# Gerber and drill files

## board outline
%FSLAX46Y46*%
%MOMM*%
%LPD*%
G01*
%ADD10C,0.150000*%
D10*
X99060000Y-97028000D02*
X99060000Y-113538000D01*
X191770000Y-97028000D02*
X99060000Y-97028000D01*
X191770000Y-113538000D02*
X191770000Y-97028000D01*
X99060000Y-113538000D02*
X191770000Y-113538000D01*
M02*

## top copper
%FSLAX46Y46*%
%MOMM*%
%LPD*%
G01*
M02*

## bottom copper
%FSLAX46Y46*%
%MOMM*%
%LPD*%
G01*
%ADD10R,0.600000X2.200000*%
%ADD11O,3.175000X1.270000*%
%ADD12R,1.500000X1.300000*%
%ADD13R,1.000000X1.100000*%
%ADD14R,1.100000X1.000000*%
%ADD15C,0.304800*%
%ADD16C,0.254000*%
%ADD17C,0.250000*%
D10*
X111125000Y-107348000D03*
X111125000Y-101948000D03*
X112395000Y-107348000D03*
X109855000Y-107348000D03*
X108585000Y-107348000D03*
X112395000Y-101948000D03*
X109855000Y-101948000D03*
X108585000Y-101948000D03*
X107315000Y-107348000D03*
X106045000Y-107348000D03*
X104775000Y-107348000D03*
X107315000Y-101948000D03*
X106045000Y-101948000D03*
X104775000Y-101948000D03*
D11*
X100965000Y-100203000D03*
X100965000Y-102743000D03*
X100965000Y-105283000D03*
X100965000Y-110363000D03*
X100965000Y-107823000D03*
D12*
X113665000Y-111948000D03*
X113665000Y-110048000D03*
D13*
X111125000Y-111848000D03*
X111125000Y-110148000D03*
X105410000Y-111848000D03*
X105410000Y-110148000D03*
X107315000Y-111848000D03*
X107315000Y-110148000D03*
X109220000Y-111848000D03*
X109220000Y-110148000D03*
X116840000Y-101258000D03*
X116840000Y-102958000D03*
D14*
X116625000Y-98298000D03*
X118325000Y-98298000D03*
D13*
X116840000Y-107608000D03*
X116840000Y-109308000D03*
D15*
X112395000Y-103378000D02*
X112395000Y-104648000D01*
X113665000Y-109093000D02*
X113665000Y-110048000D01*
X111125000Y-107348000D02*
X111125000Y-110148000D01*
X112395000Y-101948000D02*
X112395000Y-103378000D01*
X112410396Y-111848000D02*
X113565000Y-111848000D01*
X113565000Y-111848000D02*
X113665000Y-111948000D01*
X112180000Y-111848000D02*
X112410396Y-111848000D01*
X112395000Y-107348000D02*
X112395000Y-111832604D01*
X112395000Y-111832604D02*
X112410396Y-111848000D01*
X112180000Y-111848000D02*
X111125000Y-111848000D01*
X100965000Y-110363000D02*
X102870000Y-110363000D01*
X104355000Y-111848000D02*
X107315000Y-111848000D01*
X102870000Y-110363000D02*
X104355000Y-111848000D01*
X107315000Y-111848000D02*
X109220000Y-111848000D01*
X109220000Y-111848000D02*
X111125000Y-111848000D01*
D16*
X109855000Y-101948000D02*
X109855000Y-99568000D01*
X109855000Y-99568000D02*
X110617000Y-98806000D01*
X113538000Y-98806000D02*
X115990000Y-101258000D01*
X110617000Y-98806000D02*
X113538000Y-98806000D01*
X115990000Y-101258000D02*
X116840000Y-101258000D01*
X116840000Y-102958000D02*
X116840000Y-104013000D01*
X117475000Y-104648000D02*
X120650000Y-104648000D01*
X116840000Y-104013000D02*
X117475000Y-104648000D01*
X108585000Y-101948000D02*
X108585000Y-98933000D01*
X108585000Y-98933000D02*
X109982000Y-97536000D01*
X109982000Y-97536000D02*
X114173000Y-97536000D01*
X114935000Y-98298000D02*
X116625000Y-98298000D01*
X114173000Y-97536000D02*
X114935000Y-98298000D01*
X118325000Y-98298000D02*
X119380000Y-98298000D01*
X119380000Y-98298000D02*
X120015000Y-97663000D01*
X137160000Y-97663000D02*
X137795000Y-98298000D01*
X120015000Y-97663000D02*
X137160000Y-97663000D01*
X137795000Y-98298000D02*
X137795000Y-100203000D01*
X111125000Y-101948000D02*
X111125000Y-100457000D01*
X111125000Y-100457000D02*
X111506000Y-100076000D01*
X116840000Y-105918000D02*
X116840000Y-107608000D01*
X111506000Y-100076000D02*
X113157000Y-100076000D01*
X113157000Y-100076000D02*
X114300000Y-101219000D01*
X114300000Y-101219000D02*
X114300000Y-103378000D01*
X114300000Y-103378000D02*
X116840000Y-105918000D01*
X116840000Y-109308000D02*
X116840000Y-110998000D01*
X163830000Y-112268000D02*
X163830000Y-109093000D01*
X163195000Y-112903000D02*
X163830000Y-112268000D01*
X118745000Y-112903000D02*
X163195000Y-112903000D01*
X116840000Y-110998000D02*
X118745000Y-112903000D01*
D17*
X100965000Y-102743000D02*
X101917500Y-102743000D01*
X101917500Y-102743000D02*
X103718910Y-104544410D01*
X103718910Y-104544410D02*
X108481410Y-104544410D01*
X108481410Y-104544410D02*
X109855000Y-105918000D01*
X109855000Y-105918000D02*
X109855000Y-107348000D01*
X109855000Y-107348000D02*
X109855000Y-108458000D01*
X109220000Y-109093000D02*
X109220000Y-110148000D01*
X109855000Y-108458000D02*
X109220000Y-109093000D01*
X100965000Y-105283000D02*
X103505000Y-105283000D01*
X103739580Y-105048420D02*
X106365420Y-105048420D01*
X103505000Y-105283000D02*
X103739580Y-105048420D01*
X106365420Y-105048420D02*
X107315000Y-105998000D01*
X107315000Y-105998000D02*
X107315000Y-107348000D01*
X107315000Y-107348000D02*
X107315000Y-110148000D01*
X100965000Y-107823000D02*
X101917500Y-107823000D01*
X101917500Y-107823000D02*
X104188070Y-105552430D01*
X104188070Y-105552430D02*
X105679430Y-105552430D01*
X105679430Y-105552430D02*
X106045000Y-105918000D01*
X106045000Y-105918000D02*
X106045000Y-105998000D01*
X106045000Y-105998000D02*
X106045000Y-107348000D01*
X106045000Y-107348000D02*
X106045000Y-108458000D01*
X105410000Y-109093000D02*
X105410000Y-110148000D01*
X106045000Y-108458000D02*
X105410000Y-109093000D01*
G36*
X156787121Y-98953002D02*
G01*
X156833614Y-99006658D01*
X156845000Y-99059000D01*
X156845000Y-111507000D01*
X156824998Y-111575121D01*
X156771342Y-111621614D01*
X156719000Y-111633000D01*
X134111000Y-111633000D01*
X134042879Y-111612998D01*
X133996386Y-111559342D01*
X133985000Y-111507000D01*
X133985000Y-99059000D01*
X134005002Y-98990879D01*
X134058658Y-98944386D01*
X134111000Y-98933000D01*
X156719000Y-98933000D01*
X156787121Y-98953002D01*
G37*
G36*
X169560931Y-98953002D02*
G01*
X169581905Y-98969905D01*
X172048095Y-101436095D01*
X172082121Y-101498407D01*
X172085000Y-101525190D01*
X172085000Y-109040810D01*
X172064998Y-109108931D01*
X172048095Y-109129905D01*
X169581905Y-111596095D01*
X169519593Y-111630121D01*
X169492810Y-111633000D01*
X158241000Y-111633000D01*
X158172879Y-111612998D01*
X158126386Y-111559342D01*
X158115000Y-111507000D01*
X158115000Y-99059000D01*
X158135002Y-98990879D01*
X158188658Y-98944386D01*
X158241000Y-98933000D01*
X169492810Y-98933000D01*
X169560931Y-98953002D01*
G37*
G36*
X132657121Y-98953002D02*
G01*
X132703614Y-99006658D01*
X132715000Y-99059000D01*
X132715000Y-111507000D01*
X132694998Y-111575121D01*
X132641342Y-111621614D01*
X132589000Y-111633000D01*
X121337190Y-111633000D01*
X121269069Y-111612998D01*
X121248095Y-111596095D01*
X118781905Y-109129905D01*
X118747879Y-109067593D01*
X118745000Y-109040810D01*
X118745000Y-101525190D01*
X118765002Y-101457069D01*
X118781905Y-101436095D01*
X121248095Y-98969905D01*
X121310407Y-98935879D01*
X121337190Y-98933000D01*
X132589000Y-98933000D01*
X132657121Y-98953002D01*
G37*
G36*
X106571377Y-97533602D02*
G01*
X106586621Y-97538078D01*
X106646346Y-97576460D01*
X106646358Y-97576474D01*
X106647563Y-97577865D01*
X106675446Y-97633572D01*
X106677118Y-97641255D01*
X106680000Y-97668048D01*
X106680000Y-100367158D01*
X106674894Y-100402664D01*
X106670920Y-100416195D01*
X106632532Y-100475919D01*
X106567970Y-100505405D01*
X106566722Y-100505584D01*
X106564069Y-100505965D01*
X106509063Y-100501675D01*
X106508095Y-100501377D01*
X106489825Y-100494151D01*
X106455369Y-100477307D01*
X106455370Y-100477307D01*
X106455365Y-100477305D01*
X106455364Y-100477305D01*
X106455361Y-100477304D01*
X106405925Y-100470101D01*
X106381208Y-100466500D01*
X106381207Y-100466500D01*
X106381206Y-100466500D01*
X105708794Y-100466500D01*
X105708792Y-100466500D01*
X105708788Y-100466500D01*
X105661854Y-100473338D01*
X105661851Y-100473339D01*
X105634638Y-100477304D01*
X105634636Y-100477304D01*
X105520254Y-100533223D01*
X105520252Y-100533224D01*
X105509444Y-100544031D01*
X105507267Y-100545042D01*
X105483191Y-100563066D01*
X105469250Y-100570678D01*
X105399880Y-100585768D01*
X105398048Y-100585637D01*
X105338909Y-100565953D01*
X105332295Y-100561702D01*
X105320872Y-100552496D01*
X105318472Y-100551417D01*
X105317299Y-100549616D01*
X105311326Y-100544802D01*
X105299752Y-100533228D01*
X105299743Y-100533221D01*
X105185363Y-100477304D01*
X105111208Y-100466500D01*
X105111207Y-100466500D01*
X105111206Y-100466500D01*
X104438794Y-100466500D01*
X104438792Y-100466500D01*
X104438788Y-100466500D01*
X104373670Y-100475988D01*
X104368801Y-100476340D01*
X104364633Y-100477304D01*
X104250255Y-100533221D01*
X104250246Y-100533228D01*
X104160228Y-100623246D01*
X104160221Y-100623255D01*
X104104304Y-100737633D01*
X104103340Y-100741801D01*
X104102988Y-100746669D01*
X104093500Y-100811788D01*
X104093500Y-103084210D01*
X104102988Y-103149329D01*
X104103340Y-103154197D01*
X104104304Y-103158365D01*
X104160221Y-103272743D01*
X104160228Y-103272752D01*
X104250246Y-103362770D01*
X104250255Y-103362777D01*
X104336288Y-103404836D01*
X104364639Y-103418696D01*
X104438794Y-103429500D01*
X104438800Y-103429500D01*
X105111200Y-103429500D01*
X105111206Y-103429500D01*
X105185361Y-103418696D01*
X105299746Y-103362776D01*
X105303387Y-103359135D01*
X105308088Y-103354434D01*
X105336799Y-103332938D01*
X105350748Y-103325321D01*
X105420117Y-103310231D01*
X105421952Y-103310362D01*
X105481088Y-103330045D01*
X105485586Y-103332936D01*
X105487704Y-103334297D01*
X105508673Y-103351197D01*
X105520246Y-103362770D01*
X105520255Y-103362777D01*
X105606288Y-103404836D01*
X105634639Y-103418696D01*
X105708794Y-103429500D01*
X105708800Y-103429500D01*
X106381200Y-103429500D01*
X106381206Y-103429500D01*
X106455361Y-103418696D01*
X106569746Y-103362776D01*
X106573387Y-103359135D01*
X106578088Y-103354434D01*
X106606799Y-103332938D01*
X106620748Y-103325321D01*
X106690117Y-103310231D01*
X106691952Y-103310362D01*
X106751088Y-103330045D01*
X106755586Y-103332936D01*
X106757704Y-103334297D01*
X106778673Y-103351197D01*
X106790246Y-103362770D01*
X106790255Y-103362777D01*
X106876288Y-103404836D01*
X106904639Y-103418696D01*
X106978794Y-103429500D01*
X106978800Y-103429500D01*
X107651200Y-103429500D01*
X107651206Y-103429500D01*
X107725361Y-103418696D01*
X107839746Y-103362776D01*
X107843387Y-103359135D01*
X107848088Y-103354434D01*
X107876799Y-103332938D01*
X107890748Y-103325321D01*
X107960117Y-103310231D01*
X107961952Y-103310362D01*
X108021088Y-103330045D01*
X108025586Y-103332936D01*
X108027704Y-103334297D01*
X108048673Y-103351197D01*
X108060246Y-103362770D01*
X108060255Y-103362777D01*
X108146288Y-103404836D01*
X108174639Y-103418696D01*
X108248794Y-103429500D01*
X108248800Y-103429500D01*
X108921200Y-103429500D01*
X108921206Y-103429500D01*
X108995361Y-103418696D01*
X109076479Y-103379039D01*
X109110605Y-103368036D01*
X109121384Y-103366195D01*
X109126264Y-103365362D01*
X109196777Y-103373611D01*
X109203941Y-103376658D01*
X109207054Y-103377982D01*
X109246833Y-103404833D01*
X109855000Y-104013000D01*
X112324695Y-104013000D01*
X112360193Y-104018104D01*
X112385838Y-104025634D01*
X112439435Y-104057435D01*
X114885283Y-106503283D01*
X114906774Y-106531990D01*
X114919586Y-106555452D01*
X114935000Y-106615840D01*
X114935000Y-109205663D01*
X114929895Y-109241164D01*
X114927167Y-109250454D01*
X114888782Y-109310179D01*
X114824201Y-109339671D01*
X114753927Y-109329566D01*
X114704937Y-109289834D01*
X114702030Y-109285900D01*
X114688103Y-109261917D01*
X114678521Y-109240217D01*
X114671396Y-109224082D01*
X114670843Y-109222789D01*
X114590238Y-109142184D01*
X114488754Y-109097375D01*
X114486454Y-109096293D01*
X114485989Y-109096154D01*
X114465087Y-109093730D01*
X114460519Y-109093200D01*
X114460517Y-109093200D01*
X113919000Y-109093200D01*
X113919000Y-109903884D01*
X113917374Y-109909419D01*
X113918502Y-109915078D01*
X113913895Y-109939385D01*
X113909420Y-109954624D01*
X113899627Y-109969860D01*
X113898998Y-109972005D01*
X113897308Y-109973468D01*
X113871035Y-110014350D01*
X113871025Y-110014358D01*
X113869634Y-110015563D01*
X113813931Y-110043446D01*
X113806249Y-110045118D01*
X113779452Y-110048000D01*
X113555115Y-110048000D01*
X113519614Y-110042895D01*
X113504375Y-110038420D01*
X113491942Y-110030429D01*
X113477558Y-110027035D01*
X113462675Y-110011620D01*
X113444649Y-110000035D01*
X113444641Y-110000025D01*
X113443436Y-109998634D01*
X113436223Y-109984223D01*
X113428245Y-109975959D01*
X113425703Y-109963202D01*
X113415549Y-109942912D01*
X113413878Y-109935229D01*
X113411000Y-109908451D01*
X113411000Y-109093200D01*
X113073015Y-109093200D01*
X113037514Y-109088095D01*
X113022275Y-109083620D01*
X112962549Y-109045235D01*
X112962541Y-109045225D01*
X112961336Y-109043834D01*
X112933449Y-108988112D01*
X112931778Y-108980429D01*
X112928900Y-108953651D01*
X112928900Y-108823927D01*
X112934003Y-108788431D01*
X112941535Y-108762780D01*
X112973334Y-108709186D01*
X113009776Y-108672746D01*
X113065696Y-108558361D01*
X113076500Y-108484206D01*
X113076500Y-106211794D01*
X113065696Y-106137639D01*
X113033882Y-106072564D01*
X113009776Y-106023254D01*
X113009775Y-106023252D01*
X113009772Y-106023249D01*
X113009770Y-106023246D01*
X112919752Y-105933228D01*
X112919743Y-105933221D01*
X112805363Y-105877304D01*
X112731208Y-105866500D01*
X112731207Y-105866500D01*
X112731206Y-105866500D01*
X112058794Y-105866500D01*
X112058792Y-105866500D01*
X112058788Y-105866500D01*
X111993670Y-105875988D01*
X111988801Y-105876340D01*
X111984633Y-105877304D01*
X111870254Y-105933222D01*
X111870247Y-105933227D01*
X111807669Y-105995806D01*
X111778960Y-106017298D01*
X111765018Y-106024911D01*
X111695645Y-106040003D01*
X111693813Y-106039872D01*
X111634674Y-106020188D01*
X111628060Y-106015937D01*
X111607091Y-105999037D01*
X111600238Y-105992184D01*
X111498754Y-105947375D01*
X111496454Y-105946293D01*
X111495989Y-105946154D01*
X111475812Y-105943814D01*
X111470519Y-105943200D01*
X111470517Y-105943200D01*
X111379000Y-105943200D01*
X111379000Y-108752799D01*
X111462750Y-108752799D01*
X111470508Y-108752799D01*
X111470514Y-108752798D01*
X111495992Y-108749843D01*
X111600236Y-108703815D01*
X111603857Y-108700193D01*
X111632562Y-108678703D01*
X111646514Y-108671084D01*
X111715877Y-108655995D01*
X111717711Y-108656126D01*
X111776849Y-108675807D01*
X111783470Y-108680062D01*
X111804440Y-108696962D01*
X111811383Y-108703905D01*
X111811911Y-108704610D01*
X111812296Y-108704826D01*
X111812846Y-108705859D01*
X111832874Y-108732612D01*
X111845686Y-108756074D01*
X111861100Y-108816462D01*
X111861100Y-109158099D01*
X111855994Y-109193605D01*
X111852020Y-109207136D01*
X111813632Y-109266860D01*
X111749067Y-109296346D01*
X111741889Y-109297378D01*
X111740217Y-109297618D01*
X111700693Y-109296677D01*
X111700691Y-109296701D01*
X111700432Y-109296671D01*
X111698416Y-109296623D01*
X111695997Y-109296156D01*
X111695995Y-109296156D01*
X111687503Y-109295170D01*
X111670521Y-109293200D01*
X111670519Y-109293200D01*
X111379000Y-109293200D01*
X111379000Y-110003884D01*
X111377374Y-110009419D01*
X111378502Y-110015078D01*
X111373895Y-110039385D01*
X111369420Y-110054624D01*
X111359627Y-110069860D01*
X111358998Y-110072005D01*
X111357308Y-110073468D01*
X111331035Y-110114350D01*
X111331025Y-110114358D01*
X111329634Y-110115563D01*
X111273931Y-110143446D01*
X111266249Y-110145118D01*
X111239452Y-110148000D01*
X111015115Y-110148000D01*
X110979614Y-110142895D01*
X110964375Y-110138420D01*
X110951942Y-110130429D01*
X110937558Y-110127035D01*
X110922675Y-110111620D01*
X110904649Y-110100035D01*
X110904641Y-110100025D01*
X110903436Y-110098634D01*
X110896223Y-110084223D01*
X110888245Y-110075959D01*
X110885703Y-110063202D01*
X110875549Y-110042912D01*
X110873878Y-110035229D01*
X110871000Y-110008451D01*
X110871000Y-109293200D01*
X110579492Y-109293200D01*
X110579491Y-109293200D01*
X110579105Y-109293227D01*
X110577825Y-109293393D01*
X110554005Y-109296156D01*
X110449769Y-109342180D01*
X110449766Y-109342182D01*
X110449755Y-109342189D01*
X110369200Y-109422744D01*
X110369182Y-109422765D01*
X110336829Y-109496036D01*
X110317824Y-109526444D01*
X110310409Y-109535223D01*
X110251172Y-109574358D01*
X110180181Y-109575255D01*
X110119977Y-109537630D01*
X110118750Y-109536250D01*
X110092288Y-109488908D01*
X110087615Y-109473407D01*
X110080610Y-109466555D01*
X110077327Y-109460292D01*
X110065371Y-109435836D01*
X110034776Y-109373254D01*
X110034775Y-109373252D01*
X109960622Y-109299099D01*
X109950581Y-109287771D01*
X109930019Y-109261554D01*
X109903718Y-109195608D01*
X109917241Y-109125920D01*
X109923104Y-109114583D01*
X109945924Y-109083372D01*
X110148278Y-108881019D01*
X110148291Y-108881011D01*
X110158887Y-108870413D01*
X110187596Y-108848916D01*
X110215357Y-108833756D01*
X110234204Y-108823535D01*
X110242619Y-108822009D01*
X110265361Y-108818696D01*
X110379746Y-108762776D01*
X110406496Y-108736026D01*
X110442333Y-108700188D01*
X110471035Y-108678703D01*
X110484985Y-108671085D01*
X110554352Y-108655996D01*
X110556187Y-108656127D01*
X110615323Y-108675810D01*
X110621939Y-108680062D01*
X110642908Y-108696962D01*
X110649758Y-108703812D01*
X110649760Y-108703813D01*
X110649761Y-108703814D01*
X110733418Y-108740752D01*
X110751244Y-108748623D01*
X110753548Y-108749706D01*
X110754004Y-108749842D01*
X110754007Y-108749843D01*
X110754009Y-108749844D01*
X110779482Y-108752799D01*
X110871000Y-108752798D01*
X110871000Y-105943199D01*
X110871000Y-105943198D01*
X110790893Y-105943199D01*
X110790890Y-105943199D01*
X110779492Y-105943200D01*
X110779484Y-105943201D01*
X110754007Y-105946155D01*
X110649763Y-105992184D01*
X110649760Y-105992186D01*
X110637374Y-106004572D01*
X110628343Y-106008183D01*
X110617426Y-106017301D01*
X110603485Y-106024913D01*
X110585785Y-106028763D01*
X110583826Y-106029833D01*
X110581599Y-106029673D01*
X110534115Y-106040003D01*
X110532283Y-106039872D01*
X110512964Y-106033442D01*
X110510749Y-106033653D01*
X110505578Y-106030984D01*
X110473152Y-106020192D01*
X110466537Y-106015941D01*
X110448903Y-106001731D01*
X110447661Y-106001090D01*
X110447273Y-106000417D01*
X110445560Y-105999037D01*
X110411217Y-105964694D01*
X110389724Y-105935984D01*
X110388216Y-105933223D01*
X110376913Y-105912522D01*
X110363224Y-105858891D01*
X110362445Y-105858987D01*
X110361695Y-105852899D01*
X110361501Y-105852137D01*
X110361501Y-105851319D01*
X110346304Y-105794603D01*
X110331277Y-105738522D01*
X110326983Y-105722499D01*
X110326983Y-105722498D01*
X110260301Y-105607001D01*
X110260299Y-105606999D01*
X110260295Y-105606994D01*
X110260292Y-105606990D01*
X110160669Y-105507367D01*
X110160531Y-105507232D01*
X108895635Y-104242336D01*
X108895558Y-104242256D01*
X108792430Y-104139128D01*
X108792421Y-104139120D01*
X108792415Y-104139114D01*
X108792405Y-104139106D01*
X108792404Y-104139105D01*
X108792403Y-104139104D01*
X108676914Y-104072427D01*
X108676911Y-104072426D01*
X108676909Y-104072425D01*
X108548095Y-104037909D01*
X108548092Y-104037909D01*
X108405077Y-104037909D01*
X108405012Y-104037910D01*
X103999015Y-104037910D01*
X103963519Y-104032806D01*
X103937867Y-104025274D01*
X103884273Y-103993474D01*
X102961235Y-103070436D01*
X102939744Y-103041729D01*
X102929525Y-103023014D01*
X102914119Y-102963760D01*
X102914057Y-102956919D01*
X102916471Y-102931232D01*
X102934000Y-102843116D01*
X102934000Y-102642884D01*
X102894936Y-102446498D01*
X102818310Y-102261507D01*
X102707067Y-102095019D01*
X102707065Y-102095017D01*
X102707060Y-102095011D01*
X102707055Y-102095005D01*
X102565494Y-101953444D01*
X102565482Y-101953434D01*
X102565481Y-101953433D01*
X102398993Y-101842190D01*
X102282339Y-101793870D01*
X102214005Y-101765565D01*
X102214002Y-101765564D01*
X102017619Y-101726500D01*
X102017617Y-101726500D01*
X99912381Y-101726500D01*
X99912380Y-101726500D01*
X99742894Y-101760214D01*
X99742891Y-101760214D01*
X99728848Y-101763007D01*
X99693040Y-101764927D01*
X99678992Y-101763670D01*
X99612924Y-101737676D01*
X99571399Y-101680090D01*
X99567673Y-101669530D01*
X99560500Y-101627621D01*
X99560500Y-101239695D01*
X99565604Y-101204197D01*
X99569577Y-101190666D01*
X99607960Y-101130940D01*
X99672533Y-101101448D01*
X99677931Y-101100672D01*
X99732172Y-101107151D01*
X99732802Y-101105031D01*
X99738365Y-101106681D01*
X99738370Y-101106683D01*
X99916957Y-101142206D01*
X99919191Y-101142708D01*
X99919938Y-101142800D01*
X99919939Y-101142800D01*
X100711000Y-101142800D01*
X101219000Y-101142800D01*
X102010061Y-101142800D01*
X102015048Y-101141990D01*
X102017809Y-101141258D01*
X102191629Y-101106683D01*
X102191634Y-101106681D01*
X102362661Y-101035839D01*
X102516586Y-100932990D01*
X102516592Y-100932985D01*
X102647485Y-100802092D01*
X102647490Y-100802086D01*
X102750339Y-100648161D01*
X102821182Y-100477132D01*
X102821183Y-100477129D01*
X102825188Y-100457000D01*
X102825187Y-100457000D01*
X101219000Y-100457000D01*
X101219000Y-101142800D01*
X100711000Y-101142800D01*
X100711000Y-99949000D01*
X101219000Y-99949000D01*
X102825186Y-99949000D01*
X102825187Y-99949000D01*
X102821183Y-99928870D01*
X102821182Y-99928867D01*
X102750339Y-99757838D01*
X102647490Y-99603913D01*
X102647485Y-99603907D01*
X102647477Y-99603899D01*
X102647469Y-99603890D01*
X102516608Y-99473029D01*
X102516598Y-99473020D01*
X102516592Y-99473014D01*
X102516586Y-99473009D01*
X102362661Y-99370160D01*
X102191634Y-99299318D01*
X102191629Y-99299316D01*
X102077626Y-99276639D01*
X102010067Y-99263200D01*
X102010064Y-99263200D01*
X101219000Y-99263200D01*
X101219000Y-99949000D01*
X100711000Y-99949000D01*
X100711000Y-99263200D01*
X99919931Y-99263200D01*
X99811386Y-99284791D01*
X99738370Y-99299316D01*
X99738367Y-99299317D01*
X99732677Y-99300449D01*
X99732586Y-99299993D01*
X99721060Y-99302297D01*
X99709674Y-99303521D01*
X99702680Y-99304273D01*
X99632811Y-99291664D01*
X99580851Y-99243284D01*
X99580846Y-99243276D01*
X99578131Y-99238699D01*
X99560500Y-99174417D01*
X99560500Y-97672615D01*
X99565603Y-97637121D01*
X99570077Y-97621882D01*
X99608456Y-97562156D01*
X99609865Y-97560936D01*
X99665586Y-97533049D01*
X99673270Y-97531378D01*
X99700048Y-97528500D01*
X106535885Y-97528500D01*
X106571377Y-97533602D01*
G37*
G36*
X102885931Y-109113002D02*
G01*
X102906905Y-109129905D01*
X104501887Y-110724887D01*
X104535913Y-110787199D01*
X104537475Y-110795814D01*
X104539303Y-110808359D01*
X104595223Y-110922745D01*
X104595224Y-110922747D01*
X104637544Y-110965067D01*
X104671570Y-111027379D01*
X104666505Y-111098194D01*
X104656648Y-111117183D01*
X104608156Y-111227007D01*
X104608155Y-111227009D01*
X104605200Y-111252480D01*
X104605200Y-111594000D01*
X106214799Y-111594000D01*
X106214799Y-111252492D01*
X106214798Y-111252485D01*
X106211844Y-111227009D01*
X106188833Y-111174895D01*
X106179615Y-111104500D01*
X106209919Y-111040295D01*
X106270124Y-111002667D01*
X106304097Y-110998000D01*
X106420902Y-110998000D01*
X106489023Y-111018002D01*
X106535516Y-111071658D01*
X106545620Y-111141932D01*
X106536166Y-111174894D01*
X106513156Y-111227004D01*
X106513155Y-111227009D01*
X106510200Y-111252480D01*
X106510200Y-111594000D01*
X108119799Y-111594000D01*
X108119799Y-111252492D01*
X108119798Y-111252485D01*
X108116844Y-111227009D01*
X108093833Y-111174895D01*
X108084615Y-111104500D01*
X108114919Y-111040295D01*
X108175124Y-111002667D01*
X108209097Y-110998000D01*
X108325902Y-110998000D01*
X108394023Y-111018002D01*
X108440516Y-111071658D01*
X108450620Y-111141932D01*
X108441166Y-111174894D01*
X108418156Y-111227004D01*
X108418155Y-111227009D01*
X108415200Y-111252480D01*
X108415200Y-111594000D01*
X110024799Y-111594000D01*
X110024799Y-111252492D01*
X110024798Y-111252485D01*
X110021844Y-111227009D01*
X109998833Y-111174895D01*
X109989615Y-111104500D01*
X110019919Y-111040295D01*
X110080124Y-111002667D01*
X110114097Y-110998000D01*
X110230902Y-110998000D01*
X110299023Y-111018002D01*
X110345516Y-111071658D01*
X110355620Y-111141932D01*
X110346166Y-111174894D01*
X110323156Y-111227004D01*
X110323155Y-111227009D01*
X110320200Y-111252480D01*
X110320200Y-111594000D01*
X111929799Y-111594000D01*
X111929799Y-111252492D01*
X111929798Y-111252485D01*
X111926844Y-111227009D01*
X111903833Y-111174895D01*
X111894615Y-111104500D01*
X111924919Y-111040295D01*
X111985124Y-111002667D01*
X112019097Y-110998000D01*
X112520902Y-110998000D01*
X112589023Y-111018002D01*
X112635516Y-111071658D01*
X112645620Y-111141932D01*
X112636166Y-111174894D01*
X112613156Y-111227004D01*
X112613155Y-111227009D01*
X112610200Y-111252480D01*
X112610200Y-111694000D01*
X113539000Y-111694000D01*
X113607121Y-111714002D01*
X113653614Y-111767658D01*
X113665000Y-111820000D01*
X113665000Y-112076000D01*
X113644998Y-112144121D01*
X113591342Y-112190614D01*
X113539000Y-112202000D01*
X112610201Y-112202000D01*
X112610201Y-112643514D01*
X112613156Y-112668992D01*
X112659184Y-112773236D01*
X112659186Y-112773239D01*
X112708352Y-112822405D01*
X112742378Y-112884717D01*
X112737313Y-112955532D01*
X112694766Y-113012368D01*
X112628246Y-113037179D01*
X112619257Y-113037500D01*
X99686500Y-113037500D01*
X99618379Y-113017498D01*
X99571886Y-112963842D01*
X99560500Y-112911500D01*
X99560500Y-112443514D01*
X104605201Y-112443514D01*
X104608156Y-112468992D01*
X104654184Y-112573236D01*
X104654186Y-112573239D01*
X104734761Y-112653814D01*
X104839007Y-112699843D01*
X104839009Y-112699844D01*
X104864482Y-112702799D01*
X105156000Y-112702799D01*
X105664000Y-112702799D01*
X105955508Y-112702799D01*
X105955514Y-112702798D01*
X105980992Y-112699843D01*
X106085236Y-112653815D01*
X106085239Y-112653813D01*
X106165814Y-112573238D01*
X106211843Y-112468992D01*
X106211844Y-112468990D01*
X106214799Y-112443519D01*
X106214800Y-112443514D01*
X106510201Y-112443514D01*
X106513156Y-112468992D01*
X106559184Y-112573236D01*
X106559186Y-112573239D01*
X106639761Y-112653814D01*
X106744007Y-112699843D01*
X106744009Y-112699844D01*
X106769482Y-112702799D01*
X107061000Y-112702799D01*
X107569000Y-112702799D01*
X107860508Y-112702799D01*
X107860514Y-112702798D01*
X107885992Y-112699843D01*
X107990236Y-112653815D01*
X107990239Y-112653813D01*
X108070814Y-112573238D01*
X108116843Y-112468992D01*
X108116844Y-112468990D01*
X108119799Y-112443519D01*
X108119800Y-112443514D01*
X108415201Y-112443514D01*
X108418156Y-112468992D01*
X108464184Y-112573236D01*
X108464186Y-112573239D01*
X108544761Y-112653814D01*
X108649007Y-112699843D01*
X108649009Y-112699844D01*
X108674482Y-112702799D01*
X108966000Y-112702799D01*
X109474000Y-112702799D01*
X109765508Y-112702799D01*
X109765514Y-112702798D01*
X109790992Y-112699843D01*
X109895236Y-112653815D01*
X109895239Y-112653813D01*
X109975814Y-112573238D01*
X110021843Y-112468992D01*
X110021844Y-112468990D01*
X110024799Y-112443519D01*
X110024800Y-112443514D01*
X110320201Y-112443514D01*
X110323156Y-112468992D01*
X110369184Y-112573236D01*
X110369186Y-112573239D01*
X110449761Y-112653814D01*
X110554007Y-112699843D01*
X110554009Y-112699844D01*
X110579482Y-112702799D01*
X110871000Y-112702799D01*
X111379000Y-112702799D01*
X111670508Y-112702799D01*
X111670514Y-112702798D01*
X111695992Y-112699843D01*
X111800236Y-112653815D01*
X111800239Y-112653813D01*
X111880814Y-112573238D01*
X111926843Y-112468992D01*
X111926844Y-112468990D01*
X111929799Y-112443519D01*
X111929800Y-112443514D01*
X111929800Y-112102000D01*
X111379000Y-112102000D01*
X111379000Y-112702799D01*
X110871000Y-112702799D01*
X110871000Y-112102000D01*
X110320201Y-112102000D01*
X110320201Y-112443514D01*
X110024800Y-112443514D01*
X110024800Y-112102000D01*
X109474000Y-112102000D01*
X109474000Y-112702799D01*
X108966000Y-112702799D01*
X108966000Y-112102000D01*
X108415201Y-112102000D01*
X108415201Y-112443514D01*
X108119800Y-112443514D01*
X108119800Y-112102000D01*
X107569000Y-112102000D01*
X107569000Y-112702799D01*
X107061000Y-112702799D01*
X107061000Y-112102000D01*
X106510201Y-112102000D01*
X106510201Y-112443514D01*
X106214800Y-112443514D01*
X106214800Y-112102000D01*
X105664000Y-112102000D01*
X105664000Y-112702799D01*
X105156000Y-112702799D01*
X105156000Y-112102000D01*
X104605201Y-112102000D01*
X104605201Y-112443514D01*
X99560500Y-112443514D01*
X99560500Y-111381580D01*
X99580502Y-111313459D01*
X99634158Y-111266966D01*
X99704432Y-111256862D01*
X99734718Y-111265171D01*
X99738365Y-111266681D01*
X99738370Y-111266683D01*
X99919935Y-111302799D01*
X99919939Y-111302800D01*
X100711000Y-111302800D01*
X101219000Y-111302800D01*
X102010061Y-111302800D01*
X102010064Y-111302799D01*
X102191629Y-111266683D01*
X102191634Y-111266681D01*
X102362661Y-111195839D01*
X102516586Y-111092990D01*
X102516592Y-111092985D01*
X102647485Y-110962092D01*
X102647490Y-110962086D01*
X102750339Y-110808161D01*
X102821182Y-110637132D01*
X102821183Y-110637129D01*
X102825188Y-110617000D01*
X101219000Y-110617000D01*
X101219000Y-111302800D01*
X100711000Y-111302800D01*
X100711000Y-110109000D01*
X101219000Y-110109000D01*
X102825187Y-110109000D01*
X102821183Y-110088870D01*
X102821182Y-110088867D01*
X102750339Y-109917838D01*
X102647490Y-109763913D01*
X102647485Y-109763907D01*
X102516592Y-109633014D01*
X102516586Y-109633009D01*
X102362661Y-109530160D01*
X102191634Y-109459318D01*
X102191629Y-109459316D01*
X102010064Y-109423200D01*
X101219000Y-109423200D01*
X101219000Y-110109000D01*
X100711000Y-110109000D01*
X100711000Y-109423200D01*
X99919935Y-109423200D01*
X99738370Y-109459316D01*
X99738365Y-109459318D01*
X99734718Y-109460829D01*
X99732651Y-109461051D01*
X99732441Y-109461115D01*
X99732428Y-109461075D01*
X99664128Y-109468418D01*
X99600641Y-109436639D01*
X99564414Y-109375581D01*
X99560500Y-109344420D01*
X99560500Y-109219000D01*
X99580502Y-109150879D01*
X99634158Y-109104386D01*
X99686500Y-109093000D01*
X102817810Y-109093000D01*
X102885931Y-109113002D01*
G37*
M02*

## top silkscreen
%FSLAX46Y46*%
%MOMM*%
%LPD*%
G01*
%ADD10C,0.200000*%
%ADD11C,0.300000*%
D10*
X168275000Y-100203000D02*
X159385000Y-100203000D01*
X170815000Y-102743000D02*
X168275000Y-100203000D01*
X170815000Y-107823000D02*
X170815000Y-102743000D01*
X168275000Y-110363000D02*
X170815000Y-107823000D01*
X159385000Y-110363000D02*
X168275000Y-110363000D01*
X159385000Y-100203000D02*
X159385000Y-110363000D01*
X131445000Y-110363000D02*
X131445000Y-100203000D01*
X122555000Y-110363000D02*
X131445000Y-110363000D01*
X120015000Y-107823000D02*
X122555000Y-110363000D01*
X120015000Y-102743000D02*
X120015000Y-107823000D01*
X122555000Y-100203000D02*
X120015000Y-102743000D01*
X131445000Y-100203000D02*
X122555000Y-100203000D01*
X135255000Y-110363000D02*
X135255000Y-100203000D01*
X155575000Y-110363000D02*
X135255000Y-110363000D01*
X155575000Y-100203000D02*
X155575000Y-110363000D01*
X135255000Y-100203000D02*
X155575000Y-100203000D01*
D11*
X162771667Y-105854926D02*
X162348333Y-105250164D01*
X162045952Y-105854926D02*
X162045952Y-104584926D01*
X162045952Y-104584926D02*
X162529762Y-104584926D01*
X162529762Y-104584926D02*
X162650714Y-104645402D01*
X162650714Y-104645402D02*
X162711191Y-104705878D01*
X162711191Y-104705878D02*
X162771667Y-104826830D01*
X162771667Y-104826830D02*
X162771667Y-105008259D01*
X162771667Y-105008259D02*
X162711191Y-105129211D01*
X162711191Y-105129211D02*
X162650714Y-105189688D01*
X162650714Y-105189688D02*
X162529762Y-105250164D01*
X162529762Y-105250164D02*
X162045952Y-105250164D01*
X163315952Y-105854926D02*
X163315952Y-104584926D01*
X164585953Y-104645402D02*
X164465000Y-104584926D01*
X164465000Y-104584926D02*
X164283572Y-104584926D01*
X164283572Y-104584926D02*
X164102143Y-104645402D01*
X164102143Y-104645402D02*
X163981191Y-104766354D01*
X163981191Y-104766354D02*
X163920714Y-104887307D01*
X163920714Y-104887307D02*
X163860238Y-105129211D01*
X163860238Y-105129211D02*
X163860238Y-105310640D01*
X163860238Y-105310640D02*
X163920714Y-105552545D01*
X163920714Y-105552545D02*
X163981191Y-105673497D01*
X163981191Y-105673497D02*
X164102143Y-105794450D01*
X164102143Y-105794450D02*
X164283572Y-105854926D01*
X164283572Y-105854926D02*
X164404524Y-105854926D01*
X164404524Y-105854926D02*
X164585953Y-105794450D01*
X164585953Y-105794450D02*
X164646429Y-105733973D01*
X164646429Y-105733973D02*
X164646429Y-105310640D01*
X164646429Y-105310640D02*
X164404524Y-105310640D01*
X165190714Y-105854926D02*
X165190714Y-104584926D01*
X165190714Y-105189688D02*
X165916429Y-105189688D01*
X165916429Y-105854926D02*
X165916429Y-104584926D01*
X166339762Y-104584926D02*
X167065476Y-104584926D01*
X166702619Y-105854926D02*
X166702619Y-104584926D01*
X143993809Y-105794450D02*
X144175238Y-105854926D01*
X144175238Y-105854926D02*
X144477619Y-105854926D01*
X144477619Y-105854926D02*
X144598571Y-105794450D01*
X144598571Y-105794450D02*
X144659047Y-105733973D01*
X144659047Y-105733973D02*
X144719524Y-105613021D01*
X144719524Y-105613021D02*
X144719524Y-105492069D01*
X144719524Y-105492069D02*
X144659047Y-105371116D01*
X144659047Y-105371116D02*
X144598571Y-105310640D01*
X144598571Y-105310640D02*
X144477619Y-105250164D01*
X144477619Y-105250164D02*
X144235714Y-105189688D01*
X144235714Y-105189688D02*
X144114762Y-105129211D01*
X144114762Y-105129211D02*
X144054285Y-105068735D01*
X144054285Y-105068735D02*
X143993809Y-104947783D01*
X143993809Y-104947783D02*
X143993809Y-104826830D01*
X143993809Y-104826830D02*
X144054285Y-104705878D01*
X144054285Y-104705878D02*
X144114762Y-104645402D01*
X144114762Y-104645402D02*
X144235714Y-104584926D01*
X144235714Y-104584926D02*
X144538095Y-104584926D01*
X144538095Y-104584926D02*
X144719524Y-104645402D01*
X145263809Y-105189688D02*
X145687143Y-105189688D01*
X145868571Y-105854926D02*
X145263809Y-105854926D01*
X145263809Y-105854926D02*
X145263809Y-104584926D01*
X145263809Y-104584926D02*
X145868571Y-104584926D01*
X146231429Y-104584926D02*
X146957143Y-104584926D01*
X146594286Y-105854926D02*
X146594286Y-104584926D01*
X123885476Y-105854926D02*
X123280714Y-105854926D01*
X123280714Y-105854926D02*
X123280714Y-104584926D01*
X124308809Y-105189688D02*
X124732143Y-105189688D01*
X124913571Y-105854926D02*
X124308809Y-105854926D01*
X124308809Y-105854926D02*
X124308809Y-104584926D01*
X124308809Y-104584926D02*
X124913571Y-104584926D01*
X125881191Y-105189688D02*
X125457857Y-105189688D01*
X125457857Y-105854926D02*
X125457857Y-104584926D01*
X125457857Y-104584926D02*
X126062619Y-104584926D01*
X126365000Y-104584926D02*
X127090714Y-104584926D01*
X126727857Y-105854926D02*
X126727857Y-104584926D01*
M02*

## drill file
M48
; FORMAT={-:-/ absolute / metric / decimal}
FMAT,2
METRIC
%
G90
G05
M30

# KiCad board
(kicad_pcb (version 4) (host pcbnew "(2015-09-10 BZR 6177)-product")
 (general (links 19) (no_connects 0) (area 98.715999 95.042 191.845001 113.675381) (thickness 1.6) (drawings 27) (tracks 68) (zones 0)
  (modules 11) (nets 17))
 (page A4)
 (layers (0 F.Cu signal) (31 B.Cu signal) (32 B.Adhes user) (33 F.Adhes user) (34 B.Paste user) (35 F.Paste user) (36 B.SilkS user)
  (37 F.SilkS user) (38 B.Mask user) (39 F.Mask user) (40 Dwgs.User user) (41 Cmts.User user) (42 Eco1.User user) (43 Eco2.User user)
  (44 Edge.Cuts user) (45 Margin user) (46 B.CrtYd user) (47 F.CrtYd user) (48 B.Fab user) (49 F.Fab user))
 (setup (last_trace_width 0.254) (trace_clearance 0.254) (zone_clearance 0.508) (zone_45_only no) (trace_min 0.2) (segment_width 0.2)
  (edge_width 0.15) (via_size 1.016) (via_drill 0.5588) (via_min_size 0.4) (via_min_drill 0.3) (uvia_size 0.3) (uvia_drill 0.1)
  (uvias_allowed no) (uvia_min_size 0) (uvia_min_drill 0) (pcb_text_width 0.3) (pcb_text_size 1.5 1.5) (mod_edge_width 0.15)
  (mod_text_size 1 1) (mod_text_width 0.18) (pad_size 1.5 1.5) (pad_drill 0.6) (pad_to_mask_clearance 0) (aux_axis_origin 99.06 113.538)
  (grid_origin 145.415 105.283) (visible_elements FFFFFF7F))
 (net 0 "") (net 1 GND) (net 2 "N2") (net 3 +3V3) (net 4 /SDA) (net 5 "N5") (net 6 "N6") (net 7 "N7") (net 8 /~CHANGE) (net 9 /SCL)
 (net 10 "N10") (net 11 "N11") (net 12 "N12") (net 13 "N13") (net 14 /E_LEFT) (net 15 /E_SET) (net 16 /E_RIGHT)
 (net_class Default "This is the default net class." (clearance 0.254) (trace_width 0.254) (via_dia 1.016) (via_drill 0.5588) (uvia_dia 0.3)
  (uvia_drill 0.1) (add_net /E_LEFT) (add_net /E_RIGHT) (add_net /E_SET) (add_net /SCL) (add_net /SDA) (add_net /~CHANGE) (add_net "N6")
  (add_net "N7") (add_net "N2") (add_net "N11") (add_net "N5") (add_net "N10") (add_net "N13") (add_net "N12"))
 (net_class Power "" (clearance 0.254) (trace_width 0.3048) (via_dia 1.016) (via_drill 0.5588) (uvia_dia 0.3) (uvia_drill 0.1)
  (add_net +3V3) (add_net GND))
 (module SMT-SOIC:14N (layer B.Cu) (at 108.585 104.648 180)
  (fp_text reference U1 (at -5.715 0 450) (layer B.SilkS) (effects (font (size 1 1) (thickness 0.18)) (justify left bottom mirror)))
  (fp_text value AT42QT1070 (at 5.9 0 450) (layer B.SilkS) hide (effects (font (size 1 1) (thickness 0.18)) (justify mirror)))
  (pad 2 smd rect (at -2.54 -2.7 180) (size 0.6 2.2) (layers B.Cu B.Paste B.Mask) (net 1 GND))
  (pad 13 smd rect (at -2.54 2.7 180) (size 0.6 2.2) (layers B.Cu B.Paste B.Mask) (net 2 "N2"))
  (pad 1 smd rect (at -3.81 -2.7 180) (size 0.6 2.2) (layers B.Cu B.Paste B.Mask) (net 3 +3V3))
  (pad 3 smd rect (at -1.27 -2.7 180) (size 0.6 2.2) (layers B.Cu B.Paste B.Mask) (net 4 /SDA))
  (pad 4 smd rect (at 0 -2.7 180) (size 0.6 2.2) (layers B.Cu B.Paste B.Mask) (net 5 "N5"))
  (pad 14 smd rect (at -3.81 2.7 180) (size 0.6 2.2) (layers B.Cu B.Paste B.Mask) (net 1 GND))
  (pad 12 smd rect (at -1.27 2.7 180) (size 0.6 2.2) (layers B.Cu B.Paste B.Mask) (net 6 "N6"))
  (pad 11 smd rect (at 0 2.7 180) (size 0.6 2.2) (layers B.Cu B.Paste B.Mask) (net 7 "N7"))
  (pad 5 smd rect (at 1.27 -2.7 180) (size 0.6 2.2) (layers B.Cu B.Paste B.Mask) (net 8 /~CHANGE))
  (pad 6 smd rect (at 2.54 -2.7 180) (size 0.6 2.2) (layers B.Cu B.Paste B.Mask) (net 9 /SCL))
  (pad 7 smd rect (at 3.81 -2.7 180) (size 0.6 2.2) (layers B.Cu B.Paste B.Mask) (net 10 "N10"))
  (pad 10 smd rect (at 1.27 2.7 180) (size 0.6 2.2) (layers B.Cu B.Paste B.Mask) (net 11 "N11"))
  (pad 9 smd rect (at 2.54 2.7 180) (size 0.6 2.2) (layers B.Cu B.Paste B.Mask) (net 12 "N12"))
  (pad 8 smd rect (at 3.81 2.7 180) (size 0.6 2.2) (layers B.Cu B.Paste B.Mask) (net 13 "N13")))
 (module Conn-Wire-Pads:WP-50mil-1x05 (layer B.Cu) (at 100.965 105.283 270)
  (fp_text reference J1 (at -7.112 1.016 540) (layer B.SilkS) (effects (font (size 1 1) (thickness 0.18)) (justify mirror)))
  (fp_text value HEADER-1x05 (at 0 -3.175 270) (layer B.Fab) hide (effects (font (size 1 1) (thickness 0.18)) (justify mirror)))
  (pad 1 smd oval (at -5.08 0 270) (size 1.27 3.175) (layers B.Cu B.Paste B.Mask) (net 1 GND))
  (pad 2 smd oval (at -2.54 0 270) (size 1.27 3.175) (layers B.Cu B.Paste B.Mask) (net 4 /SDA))
  (pad 3 smd oval (at 0 0 270) (size 1.27 3.175) (layers B.Cu B.Paste B.Mask) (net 8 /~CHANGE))
  (pad 5 smd oval (at 5.08 0 270) (size 1.27 3.175) (layers B.Cu B.Paste B.Mask) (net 3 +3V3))
  (pad 4 smd oval (at 2.54 0 270) (size 1.27 3.175) (layers B.Cu B.Paste B.Mask) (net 9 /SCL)))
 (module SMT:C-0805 (layer B.Cu) (at 113.665 110.998 90)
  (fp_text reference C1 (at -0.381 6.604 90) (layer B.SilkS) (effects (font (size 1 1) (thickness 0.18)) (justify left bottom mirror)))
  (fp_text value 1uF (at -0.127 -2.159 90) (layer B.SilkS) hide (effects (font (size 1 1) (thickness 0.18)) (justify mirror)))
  (pad 1 smd rect (at -0.95 0 90) (size 1.3 1.5) (layers B.Cu B.Paste B.Mask) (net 3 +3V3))
  (pad 2 smd rect (at 0.95 0 90) (size 1.3 1.5) (layers B.Cu B.Paste B.Mask) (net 1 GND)))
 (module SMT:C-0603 (layer B.Cu) (at 111.125 110.998 90)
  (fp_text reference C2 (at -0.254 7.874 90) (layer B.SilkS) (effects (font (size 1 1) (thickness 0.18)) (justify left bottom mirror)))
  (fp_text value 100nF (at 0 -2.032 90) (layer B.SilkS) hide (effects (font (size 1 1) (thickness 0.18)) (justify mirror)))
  (pad 1 smd rect (at -0.85 0 90) (size 1.1 1) (layers B.Cu B.Paste B.Mask) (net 3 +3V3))
  (pad 2 smd rect (at 0.85 0 90) (size 1.1 1) (layers B.Cu B.Paste B.Mask) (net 1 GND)))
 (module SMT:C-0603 (layer B.Cu) (at 105.41 110.998 90)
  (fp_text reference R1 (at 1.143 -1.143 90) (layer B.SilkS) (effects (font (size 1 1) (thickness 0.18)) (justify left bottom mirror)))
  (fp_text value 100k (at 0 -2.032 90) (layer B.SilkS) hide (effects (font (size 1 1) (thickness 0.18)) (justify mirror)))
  (pad 1 smd rect (at -0.85 0 90) (size 1.1 1) (layers B.Cu B.Paste B.Mask) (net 3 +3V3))
  (pad 2 smd rect (at 0.85 0 90) (size 1.1 1) (layers B.Cu B.Paste B.Mask) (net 9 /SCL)))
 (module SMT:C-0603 (layer B.Cu) (at 107.315 110.998 90)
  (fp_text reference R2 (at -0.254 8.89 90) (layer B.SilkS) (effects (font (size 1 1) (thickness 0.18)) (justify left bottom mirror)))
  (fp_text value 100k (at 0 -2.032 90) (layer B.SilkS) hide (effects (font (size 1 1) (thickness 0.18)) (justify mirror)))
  (pad 1 smd rect (at -0.85 0 90) (size 1.1 1) (layers B.Cu B.Paste B.Mask) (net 3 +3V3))
  (pad 2 smd rect (at 0.85 0 90) (size 1.1 1) (layers B.Cu B.Paste B.Mask) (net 8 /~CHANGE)))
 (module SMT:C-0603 (layer B.Cu) (at 109.22 110.998 90)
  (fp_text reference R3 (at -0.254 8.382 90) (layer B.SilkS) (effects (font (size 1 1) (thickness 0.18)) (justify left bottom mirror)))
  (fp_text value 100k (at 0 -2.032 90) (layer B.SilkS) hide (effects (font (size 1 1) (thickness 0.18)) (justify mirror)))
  (pad 1 smd rect (at -0.85 0 90) (size 1.1 1) (layers B.Cu B.Paste B.Mask) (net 3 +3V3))
  (pad 2 smd rect (at 0.85 0 90) (size 1.1 1) (layers B.Cu B.Paste B.Mask) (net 4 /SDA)))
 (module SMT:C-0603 (layer B.Cu) (at 116.84 102.108 270)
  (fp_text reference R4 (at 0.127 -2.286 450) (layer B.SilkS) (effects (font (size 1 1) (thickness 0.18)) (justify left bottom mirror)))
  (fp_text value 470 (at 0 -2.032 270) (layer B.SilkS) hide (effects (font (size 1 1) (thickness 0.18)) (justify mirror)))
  (pad 1 smd rect (at -0.85 0 270) (size 1.1 1) (layers B.Cu B.Paste B.Mask) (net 6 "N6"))
  (pad 2 smd rect (at 0.85 0 270) (size 1.1 1) (layers B.Cu B.Paste B.Mask) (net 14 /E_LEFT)))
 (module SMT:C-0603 (layer B.Cu) (at 117.475 98.298)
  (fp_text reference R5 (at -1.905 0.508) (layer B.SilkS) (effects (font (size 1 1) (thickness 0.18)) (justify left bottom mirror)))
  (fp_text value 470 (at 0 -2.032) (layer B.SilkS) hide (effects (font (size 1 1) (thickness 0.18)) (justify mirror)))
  (pad 1 smd rect (at -0.85 0) (size 1.1 1) (layers B.Cu B.Paste B.Mask) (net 7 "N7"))
  (pad 2 smd rect (at 0.85 0) (size 1.1 1) (layers B.Cu B.Paste B.Mask) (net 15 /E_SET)))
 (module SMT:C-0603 (layer B.Cu) (at 116.84 108.458 270)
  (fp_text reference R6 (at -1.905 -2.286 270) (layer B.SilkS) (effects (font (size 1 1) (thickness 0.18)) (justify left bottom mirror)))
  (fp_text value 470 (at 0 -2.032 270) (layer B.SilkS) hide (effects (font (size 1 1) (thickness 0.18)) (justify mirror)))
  (pad 1 smd rect (at -0.85 0 270) (size 1.1 1) (layers B.Cu B.Paste B.Mask) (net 2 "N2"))
  (pad 2 smd rect (at 0.85 0 270) (size 1.1 1) (layers B.Cu B.Paste B.Mask) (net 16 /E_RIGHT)))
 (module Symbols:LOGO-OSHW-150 (layer B.Cu) (at 175.133 107.823 180)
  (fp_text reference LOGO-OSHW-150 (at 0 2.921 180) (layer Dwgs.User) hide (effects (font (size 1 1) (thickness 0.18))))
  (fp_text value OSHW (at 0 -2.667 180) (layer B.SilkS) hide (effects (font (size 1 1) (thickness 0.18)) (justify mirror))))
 (gr_line (start 168.275 100.203) (end 159.385 100.203) (angle 90) (layer F.SilkS) (width 0.2))
 (gr_line (start 170.815 102.743) (end 168.275 100.203) (angle 90) (layer F.SilkS) (width 0.2))
 (gr_line (start 170.815 107.823) (end 170.815 102.743) (angle 90) (layer F.SilkS) (width 0.2))
 (gr_line (start 168.275 110.363) (end 170.815 107.823) (angle 90) (layer F.SilkS) (width 0.2))
 (gr_line (start 159.385 110.363) (end 168.275 110.363) (angle 90) (layer F.SilkS) (width 0.2))
 (gr_line (start 159.385 100.203) (end 159.385 110.363) (angle 90) (layer F.SilkS) (width 0.2))
 (gr_line (start 131.445 110.363) (end 131.445 100.203) (angle 90) (layer F.SilkS) (width 0.2))
 (gr_line (start 122.555 110.363) (end 131.445 110.363) (angle 90) (layer F.SilkS) (width 0.2))
 (gr_line (start 120.015 107.823) (end 122.555 110.363) (angle 90) (layer F.SilkS) (width 0.2))
 (gr_line (start 120.015 102.743) (end 120.015 107.823) (angle 90) (layer F.SilkS) (width 0.2))
 (gr_line (start 122.555 100.203) (end 120.015 102.743) (angle 90) (layer F.SilkS) (width 0.2))
 (gr_line (start 131.445 100.203) (end 122.555 100.203) (angle 90) (layer F.SilkS) (width 0.2))
 (gr_line (start 135.255 110.363) (end 135.255 100.203) (angle 90) (layer F.SilkS) (width 0.2))
 (gr_line (start 155.575 110.363) (end 135.255 110.363) (angle 90) (layer F.SilkS) (width 0.2))
 (gr_line (start 155.575 100.203) (end 155.575 110.363) (angle 90) (layer F.SilkS) (width 0.2))
 (gr_line (start 135.255 100.203) (end 155.575 100.203) (angle 90) (layer F.SilkS) (width 0.2))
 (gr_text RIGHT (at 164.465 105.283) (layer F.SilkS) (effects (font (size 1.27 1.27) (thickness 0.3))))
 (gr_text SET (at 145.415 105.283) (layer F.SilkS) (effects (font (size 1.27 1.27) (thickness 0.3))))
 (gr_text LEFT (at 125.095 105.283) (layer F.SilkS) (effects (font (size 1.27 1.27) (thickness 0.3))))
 (gr_line (start 99.06 97.028) (end 99.06 113.538) (angle 90) (layer Edge.Cuts) (width 0.15))
 (gr_line (start 191.77 97.028) (end 99.06 97.028) (angle 90) (layer Edge.Cuts) (width 0.15))
 (gr_line (start 191.77 113.538) (end 191.77 97.028) (angle 90) (layer Edge.Cuts) (width 0.15))
 (gr_line (start 99.06 113.538) (end 191.77 113.538) (angle 90) (layer Edge.Cuts) (width 0.15))
 (segment (start 112.395 103.378) (end 112.395 104.648) (width 0.3048) (layer B.Cu) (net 1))
 (segment (start 113.665 109.093) (end 113.665 110.048) (width 0.3048) (layer B.Cu) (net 1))
 (segment (start 111.125 107.348) (end 111.125 110.148) (width 0.3048) (layer B.Cu) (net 1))
 (segment (start 112.395 101.948) (end 112.395 103.378) (width 0.3048) (layer B.Cu) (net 1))
 (segment (start 112.410396 111.848) (end 113.565 111.848) (width 0.3048) (layer B.Cu) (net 3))
 (segment (start 113.565 111.848) (end 113.665 111.948) (width 0.3048) (layer B.Cu) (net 3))
 (segment (start 112.18 111.848) (end 112.410396 111.848) (width 0.3048) (layer B.Cu) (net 3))
 (segment (start 112.395 107.348) (end 112.395 111.832604) (width 0.3048) (layer B.Cu) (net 3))
 (segment (start 112.395 111.832604) (end 112.410396 111.848) (width 0.3048) (layer B.Cu) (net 3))
 (segment (start 112.18 111.848) (end 111.125 111.848) (width 0.3048) (layer B.Cu) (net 3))
 (segment (start 100.965 110.363) (end 102.87 110.363) (width 0.3048) (layer B.Cu) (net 3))
 (segment (start 104.355 111.848) (end 107.315 111.848) (width 0.3048) (layer B.Cu) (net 3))
 (segment (start 102.87 110.363) (end 104.355 111.848) (width 0.3048) (layer B.Cu) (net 3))
 (segment (start 107.315 111.848) (end 109.22 111.848) (width 0.3048) (layer B.Cu) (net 3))
 (segment (start 109.22 111.848) (end 111.125 111.848) (width 0.3048) (layer B.Cu) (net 3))
 (segment (start 109.855 101.948) (end 109.855 99.568) (width 0.254) (layer B.Cu) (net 6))
 (segment (start 109.855 99.568) (end 110.617 98.806) (width 0.254) (layer B.Cu) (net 6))
 (segment (start 113.538 98.806) (end 115.99 101.258) (width 0.254) (layer B.Cu) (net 6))
 (segment (start 110.617 98.806) (end 113.538 98.806) (width 0.254) (layer B.Cu) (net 6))
 (segment (start 115.99 101.258) (end 116.84 101.258) (width 0.254) (layer B.Cu) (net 6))
 (segment (start 116.84 102.958) (end 116.84 104.013) (width 0.254) (layer B.Cu) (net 14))
 (segment (start 117.475 104.648) (end 120.65 104.648) (width 0.254) (layer B.Cu) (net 14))
 (segment (start 116.84 104.013) (end 117.475 104.648) (width 0.254) (layer B.Cu) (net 14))
 (segment (start 108.585 101.948) (end 108.585 98.933) (width 0.254) (layer B.Cu) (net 7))
 (segment (start 108.585 98.933) (end 109.982 97.536) (width 0.254) (layer B.Cu) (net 7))
 (segment (start 109.982 97.536) (end 114.173 97.536) (width 0.254) (layer B.Cu) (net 7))
 (segment (start 114.935 98.298) (end 116.625 98.298) (width 0.254) (layer B.Cu) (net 7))
 (segment (start 114.173 97.536) (end 114.935 98.298) (width 0.254) (layer B.Cu) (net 7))
 (segment (start 118.325 98.298) (end 119.38 98.298) (width 0.254) (layer B.Cu) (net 15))
 (segment (start 119.38 98.298) (end 120.015 97.663) (width 0.254) (layer B.Cu) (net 15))
 (segment (start 137.16 97.663) (end 137.795 98.298) (width 0.254) (layer B.Cu) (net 15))
 (segment (start 120.015 97.663) (end 137.16 97.663) (width 0.254) (layer B.Cu) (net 15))
 (segment (start 137.795 98.298) (end 137.795 100.203) (width 0.254) (layer B.Cu) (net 15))
 (segment (start 111.125 101.948) (end 111.125 100.457) (width 0.254) (layer B.Cu) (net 2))
 (segment (start 111.125 100.457) (end 111.506 100.076) (width 0.254) (layer B.Cu) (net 2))
 (segment (start 116.84 105.918) (end 116.84 107.608) (width 0.254) (layer B.Cu) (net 2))
 (segment (start 111.506 100.076) (end 113.157 100.076) (width 0.254) (layer B.Cu) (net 2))
 (segment (start 113.157 100.076) (end 114.3 101.219) (width 0.254) (layer B.Cu) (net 2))
 (segment (start 114.3 101.219) (end 114.3 103.378) (width 0.254) (layer B.Cu) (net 2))
 (segment (start 114.3 103.378) (end 116.84 105.918) (width 0.254) (layer B.Cu) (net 2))
 (segment (start 116.84 109.308) (end 116.84 110.998) (width 0.254) (layer B.Cu) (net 16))
 (segment (start 163.83 112.268) (end 163.83 109.093) (width 0.254) (layer B.Cu) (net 16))
 (segment (start 163.195 112.903) (end 163.83 112.268) (width 0.254) (layer B.Cu) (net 16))
 (segment (start 118.745 112.903) (end 163.195 112.903) (width 0.254) (layer B.Cu) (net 16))
 (segment (start 116.84 110.998) (end 118.745 112.903) (width 0.254) (layer B.Cu) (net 16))
 (segment (start 100.965 102.743) (end 101.9175 102.743) (width 0.25) (layer B.Cu) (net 4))
 (segment (start 101.9175 102.743) (end 103.71891 104.54441) (width 0.25) (layer B.Cu) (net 4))
 (segment (start 103.71891 104.54441) (end 108.48141 104.54441) (width 0.25) (layer B.Cu) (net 4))
 (segment (start 108.48141 104.54441) (end 109.855 105.918) (width 0.25) (layer B.Cu) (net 4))
 (segment (start 109.855 105.918) (end 109.855 107.348) (width 0.25) (layer B.Cu) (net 4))
 (segment (start 109.855 107.348) (end 109.855 108.458) (width 0.25) (layer B.Cu) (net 4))
 (segment (start 109.22 109.093) (end 109.22 110.148) (width 0.25) (layer B.Cu) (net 4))
 (segment (start 109.855 108.458) (end 109.22 109.093) (width 0.25) (layer B.Cu) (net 4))
 (segment (start 100.965 105.283) (end 103.505 105.283) (width 0.25) (layer B.Cu) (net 8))
 (segment (start 103.73958 105.04842) (end 106.36542 105.04842) (width 0.25) (layer B.Cu) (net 8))
 (segment (start 103.505 105.283) (end 103.73958 105.04842) (width 0.25) (layer B.Cu) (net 8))
 (segment (start 106.36542 105.04842) (end 107.315 105.998) (width 0.25) (layer B.Cu) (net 8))
 (segment (start 107.315 105.998) (end 107.315 107.348) (width 0.25) (layer B.Cu) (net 8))
 (segment (start 107.315 107.348) (end 107.315 110.148) (width 0.25) (layer B.Cu) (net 8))
 (segment (start 100.965 107.823) (end 101.9175 107.823) (width 0.25) (layer B.Cu) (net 9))
 (segment (start 101.9175 107.823) (end 104.18807 105.55243) (width 0.25) (layer B.Cu) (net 9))
 (segment (start 104.18807 105.55243) (end 105.67943 105.55243) (width 0.25) (layer B.Cu) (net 9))
 (segment (start 105.67943 105.55243) (end 106.045 105.918) (width 0.25) (layer B.Cu) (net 9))
 (segment (start 106.045 105.918) (end 106.045 105.998) (width 0.25) (layer B.Cu) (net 9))
 (segment (start 106.045 105.998) (end 106.045 107.348) (width 0.25) (layer B.Cu) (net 9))
 (segment (start 106.045 107.348) (end 106.045 108.458) (width 0.25) (layer B.Cu) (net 9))
 (segment (start 105.41 109.093) (end 105.41 110.148) (width 0.25) (layer B.Cu) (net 9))
 (segment (start 106.045 108.458) (end 105.41 109.093) (width 0.25) (layer B.Cu) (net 9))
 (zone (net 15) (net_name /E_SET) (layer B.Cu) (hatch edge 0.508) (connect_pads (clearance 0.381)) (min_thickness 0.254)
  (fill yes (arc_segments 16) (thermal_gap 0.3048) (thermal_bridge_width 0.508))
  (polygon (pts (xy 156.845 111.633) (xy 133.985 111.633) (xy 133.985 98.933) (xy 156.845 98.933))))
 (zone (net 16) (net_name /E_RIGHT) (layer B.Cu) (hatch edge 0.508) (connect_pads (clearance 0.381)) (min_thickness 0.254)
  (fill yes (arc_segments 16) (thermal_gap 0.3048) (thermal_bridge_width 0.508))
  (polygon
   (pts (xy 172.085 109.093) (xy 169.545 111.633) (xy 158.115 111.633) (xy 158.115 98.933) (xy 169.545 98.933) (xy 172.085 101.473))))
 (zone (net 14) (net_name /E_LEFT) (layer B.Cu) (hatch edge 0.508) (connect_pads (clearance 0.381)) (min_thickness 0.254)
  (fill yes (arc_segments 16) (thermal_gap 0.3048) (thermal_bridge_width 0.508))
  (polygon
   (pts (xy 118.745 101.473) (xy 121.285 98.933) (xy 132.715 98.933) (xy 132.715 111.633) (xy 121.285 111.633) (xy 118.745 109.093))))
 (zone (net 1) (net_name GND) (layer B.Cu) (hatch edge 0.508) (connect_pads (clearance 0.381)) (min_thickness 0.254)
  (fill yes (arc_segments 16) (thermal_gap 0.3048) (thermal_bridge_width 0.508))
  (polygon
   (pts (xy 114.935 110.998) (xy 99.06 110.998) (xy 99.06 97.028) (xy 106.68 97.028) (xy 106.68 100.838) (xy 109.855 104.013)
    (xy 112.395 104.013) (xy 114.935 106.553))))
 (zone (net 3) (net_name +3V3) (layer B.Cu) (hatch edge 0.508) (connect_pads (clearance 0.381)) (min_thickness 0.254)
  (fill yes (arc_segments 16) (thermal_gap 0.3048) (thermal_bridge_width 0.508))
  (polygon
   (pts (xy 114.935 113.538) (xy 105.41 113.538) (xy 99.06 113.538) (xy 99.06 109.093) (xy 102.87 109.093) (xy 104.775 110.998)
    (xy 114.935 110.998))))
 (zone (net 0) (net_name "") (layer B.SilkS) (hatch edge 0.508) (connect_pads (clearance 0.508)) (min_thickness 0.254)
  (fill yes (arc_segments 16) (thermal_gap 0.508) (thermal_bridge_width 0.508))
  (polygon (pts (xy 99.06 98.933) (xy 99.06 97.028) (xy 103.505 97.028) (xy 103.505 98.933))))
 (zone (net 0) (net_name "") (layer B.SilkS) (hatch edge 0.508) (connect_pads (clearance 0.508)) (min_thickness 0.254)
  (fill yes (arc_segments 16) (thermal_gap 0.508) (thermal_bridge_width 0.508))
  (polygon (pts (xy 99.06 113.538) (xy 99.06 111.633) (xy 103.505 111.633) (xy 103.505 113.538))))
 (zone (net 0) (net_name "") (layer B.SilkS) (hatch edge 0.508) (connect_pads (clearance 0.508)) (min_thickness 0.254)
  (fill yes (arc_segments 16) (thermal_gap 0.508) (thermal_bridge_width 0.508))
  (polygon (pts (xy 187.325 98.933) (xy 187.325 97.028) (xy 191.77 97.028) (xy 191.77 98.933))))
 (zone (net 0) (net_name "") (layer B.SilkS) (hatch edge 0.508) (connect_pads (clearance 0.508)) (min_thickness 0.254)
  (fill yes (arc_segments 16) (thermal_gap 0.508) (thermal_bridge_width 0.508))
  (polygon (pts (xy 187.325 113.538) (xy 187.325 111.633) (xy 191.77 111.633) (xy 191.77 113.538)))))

